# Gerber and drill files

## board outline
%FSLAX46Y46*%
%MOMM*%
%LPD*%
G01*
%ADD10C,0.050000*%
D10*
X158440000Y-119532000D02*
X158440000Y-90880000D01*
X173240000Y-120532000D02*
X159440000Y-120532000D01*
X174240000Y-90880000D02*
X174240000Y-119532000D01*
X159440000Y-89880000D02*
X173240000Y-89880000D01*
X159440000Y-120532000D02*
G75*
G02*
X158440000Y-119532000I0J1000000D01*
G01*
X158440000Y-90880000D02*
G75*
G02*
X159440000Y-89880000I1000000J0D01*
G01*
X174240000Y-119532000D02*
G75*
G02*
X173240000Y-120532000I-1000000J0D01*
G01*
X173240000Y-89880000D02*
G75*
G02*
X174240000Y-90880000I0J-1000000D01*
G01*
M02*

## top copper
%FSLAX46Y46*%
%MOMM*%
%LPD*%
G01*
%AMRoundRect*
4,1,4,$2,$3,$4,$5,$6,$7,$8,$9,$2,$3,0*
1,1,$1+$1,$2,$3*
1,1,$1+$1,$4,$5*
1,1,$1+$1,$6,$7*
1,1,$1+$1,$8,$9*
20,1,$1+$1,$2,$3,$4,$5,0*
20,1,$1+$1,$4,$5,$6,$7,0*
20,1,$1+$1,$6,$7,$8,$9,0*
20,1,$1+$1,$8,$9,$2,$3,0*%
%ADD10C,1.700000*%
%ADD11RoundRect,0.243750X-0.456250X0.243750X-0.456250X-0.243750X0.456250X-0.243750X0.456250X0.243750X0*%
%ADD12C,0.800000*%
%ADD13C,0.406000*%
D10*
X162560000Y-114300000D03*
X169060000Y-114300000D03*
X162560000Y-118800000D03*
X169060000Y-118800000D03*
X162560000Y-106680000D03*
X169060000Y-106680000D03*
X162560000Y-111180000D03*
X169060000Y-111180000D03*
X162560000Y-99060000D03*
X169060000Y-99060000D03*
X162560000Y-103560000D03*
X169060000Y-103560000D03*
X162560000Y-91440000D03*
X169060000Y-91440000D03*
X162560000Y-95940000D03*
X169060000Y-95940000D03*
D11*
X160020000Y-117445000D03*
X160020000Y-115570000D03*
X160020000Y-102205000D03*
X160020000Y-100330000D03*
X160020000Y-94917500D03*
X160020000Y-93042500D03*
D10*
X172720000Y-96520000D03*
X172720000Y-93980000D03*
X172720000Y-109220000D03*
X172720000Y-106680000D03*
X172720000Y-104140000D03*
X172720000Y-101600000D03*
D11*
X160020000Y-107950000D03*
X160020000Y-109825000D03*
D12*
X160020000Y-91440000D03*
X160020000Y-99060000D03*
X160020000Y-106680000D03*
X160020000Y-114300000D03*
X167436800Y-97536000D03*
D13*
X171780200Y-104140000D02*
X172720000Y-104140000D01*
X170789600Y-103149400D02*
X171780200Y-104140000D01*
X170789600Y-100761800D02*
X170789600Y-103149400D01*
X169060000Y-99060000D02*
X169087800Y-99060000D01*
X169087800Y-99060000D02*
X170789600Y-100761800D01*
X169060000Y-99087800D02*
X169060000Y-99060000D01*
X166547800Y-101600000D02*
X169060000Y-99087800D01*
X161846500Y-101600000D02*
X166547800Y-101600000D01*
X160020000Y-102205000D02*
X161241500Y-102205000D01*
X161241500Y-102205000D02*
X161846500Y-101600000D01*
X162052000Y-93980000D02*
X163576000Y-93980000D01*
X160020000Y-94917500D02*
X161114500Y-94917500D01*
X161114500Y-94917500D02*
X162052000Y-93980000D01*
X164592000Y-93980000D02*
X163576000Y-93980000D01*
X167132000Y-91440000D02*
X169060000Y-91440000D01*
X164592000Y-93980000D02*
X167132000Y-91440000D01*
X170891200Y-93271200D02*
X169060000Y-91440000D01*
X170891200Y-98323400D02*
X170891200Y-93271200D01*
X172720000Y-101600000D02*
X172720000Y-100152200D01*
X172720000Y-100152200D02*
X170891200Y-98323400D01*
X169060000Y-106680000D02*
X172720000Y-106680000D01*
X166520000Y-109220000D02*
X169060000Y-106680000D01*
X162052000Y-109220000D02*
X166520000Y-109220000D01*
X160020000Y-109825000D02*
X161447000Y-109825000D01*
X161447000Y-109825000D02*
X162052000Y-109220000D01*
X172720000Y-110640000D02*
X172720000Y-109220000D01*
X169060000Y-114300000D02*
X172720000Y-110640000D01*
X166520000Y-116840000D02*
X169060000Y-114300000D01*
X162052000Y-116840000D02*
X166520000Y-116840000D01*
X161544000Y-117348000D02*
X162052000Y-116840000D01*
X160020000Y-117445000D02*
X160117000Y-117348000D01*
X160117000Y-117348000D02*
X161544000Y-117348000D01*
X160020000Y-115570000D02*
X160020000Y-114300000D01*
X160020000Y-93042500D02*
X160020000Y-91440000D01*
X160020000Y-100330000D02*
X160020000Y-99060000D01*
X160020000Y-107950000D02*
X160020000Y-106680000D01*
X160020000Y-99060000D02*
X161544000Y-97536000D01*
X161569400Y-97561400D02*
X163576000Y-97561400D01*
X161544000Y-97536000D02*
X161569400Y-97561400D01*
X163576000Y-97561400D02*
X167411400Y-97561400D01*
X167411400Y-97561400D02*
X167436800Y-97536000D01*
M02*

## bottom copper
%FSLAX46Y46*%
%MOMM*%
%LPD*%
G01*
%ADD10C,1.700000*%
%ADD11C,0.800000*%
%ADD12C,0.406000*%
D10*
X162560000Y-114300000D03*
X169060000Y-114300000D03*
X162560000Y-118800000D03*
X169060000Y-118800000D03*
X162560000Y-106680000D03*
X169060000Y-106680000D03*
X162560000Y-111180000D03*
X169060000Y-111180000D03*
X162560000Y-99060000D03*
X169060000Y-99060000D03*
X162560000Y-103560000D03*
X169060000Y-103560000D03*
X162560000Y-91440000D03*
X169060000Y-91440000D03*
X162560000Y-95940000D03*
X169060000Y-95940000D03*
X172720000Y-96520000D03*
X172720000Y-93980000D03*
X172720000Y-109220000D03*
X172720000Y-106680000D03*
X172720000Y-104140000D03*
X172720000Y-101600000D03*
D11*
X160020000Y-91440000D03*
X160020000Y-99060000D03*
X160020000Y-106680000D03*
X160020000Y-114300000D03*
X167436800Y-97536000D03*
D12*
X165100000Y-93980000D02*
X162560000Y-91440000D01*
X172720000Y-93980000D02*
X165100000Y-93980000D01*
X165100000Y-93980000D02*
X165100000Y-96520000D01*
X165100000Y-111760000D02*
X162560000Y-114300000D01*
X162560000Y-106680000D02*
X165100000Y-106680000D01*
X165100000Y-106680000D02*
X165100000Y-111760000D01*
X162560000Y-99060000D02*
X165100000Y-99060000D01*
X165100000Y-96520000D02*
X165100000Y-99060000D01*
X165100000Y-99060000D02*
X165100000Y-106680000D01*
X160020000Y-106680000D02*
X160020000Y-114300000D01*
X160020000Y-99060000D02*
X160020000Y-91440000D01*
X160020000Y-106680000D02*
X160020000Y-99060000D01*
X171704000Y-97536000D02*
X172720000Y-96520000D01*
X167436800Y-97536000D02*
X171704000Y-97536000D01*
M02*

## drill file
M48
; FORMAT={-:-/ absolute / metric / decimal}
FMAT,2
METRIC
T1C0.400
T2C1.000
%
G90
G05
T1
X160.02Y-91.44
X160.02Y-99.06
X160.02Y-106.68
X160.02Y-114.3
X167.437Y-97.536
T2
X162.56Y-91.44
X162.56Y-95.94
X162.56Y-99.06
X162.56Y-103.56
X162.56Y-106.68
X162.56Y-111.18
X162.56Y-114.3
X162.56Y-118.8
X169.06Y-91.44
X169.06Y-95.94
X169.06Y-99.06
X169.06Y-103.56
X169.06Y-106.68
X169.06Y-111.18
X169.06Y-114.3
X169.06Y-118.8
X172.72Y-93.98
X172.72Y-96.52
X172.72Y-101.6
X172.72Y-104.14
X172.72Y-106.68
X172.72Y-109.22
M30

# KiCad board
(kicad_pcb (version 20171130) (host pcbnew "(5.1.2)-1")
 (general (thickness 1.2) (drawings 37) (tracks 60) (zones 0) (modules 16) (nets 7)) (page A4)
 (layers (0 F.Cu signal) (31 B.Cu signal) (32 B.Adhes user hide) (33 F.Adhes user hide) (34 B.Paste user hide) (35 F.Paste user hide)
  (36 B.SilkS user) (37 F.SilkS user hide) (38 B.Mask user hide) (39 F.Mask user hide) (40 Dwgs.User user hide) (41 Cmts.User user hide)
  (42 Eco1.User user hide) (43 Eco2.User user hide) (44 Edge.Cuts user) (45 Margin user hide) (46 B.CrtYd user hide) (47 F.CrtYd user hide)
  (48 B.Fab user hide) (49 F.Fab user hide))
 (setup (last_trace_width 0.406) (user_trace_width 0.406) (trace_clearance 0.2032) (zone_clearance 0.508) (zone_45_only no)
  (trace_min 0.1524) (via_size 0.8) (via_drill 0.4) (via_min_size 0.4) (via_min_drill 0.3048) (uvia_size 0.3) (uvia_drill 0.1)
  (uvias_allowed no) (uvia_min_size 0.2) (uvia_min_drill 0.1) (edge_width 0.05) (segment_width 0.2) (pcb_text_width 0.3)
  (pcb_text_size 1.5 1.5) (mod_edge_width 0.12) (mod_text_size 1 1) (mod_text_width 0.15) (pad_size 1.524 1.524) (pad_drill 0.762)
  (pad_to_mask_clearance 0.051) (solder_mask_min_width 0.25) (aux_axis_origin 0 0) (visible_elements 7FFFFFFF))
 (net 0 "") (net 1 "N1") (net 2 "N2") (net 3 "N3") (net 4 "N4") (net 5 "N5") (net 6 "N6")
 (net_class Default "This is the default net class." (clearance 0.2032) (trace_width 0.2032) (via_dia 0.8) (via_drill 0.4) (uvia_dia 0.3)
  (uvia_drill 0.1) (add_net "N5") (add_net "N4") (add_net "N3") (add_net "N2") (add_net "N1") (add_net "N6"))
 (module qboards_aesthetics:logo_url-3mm (layer B.Cu) (at 165.2778 94.742 270)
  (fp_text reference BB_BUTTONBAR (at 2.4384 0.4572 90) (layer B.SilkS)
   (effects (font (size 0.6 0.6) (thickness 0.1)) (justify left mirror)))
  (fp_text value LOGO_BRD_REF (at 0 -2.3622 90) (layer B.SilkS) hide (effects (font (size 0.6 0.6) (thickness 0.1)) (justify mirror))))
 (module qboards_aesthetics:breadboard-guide (layer F.Cu) (at 137.16 93.98)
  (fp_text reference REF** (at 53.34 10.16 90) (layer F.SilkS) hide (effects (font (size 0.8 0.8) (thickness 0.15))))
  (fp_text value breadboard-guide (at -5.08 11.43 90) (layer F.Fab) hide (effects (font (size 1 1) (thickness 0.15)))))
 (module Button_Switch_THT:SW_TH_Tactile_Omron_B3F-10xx (layer F.Cu) (at 162.56 114.3)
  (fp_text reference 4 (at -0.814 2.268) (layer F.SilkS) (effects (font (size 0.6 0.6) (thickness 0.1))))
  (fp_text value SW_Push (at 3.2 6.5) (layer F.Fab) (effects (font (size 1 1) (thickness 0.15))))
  (pad 1 thru_hole circle (at 0 0) (size 1.7 1.7) (drill 1) (layers *.Cu *.Mask) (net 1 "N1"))
  (pad 2 thru_hole circle (at 6.5 0) (size 1.7 1.7) (drill 1) (layers *.Cu *.Mask) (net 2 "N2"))
  (pad 3 thru_hole circle (at 0 4.5) (size 1.7 1.7) (drill 1) (layers *.Cu *.Mask))
  (pad 4 thru_hole circle (at 6.5 4.5) (size 1.7 1.7) (drill 1) (layers *.Cu *.Mask)))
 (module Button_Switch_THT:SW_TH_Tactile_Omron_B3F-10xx (layer F.Cu) (at 162.56 106.68)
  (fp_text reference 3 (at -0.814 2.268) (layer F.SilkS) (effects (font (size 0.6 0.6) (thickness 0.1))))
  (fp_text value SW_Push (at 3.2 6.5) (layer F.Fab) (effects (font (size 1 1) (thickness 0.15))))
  (pad 1 thru_hole circle (at 0 0) (size 1.7 1.7) (drill 1) (layers *.Cu *.Mask) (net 1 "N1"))
  (pad 2 thru_hole circle (at 6.5 0) (size 1.7 1.7) (drill 1) (layers *.Cu *.Mask) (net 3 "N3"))
  (pad 3 thru_hole circle (at 0 4.5) (size 1.7 1.7) (drill 1) (layers *.Cu *.Mask))
  (pad 4 thru_hole circle (at 6.5 4.5) (size 1.7 1.7) (drill 1) (layers *.Cu *.Mask)))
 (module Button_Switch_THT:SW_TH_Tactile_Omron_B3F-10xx (layer F.Cu) (at 162.56 99.06)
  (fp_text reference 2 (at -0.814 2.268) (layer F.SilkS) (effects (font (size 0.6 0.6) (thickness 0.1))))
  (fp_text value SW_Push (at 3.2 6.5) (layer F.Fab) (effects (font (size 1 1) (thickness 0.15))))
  (pad 1 thru_hole circle (at 0 0) (size 1.7 1.7) (drill 1) (layers *.Cu *.Mask) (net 1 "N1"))
  (pad 2 thru_hole circle (at 6.5 0) (size 1.7 1.7) (drill 1) (layers *.Cu *.Mask) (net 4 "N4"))
  (pad 3 thru_hole circle (at 0 4.5) (size 1.7 1.7) (drill 1) (layers *.Cu *.Mask))
  (pad 4 thru_hole circle (at 6.5 4.5) (size 1.7 1.7) (drill 1) (layers *.Cu *.Mask)))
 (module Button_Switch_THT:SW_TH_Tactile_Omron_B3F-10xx (layer F.Cu) (at 162.56 91.44)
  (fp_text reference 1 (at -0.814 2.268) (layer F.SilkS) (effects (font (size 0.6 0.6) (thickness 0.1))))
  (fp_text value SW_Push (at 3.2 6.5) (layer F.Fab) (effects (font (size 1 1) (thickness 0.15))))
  (pad 1 thru_hole circle (at 0 0) (size 1.7 1.7) (drill 1) (layers *.Cu *.Mask) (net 1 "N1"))
  (pad 2 thru_hole circle (at 6.5 0) (size 1.7 1.7) (drill 1) (layers *.Cu *.Mask) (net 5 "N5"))
  (pad 3 thru_hole circle (at 0 4.5) (size 1.7 1.7) (drill 1) (layers *.Cu *.Mask))
  (pad 4 thru_hole circle (at 6.5 4.5) (size 1.7 1.7) (drill 1) (layers *.Cu *.Mask)))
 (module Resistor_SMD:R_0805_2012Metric (layer F.Cu) (at 160.02 116.5075 270)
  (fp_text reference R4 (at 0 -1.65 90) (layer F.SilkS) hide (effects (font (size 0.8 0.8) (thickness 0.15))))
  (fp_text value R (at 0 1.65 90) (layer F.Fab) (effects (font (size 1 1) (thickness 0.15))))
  (pad 2 smd roundrect (at 0.9375 0 270) (size 0.975 1.4) (layers F.Cu F.Paste F.Mask) (roundrect_rratio 0.25) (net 2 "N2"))
  (pad 1 smd roundrect (at -0.9375 0 270) (size 0.975 1.4) (layers F.Cu F.Paste F.Mask) (roundrect_rratio 0.25) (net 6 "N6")))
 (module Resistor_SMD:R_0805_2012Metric (layer F.Cu) (at 160.02 101.2675 270)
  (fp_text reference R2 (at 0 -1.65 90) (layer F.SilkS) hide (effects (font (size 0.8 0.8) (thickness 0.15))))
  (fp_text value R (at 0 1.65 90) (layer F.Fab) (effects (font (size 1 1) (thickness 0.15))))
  (pad 2 smd roundrect (at 0.9375 0 270) (size 0.975 1.4) (layers F.Cu F.Paste F.Mask) (roundrect_rratio 0.25) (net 4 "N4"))
  (pad 1 smd roundrect (at -0.9375 0 270) (size 0.975 1.4) (layers F.Cu F.Paste F.Mask) (roundrect_rratio 0.25) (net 6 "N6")))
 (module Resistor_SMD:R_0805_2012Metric (layer F.Cu) (at 160.02 93.98 270)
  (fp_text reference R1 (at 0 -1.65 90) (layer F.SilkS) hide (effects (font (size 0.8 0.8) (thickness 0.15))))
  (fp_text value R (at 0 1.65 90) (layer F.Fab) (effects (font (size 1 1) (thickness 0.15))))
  (pad 2 smd roundrect (at 0.9375 0 270) (size 0.975 1.4) (layers F.Cu F.Paste F.Mask) (roundrect_rratio 0.25) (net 5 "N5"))
  (pad 1 smd roundrect (at -0.9375 0 270) (size 0.975 1.4) (layers F.Cu F.Paste F.Mask) (roundrect_rratio 0.25) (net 6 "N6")))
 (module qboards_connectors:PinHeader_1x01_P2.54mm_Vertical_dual (layer F.Cu) (at 172.72 96.52)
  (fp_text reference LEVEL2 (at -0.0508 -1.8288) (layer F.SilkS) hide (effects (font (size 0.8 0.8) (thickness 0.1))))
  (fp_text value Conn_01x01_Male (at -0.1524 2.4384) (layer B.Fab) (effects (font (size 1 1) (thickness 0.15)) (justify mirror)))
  (pad 1 thru_hole circle (at 0 0) (size 1.7 1.7) (drill 1) (layers *.Cu *.Mask) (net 6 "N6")))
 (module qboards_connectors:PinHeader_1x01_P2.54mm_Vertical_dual (layer F.Cu) (at 172.72 93.98)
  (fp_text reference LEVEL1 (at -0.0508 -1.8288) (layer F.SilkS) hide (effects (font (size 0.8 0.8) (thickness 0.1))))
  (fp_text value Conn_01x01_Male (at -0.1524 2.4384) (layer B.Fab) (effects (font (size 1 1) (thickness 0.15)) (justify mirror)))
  (pad 1 thru_hole circle (at 0 0) (size 1.7 1.7) (drill 1) (layers *.Cu *.Mask) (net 1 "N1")))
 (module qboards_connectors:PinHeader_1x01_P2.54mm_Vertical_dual (layer F.Cu) (at 172.72 109.22)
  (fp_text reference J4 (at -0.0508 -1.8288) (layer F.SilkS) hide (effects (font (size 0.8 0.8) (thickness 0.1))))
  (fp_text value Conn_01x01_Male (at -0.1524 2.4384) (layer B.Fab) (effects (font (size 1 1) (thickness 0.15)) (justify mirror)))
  (pad 1 thru_hole circle (at 0 0) (size 1.7 1.7) (drill 1) (layers *.Cu *.Mask) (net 2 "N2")))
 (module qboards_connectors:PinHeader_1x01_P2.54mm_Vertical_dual (layer F.Cu) (at 172.72 106.68)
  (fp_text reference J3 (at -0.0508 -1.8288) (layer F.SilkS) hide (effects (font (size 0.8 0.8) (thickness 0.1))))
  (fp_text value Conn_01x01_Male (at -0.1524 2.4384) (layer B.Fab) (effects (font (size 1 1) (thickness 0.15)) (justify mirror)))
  (pad 1 thru_hole circle (at 0 0) (size 1.7 1.7) (drill 1) (layers *.Cu *.Mask) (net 3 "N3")))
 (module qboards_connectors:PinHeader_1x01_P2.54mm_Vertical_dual (layer F.Cu) (at 172.72 104.14)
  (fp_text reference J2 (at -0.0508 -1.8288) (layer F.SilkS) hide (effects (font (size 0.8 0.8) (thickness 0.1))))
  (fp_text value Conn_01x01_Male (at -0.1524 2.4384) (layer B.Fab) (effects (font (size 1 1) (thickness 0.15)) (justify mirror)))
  (pad 1 thru_hole circle (at 0 0) (size 1.7 1.7) (drill 1) (layers *.Cu *.Mask) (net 4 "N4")))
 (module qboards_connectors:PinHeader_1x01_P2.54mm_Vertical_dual (layer F.Cu) (at 172.72 101.6)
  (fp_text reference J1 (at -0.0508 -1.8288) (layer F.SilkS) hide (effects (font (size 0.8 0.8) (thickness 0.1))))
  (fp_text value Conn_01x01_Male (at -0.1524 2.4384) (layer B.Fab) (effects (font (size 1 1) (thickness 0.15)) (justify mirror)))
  (pad 1 thru_hole circle (at 0 0) (size 1.7 1.7) (drill 1) (layers *.Cu *.Mask) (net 5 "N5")))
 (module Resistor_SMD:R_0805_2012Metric (layer F.Cu) (at 160.02 108.8875 270)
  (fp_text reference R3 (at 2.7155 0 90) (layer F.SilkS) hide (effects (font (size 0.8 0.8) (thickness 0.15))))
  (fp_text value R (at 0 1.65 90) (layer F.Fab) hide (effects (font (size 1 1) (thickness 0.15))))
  (pad 1 smd roundrect (at -0.9375 0 270) (size 0.975 1.4) (layers F.Cu F.Paste F.Mask) (roundrect_rratio 0.25) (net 6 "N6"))
  (pad 2 smd roundrect (at 0.9375 0 270) (size 0.975 1.4) (layers F.Cu F.Paste F.Mask) (roundrect_rratio 0.25) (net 3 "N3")))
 (gr_line (start 158.44 119.532) (end 158.44 90.88) (layer Edge.Cuts) (width 0.05))
 (gr_line (start 173.24 120.532) (end 159.44 120.532) (layer Edge.Cuts) (width 0.05))
 (gr_line (start 174.24 90.88) (end 174.24 119.532) (layer Edge.Cuts) (width 0.05))
 (gr_line (start 159.44 89.88) (end 173.24 89.88) (layer Edge.Cuts) (width 0.05))
 (gr_arc (start 159.44 119.532) (end 158.44 119.532) (angle -90) (layer Edge.Cuts) (width 0.05))
 (gr_arc (start 159.44 90.88) (end 159.44 89.88) (angle -90) (layer Edge.Cuts) (width 0.05))
 (gr_arc (start 173.24 119.532) (end 173.24 120.532) (angle -90) (layer Edge.Cuts) (width 0.05))
 (gr_arc (start 173.24 90.88) (end 174.24 90.88) (angle -90) (layer Edge.Cuts) (width 0.05))
 (segment (start 171.7802 104.14) (end 172.72 104.14) (width 0.406) (layer F.Cu) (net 4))
 (segment (start 170.7896 103.1494) (end 171.7802 104.14) (width 0.406) (layer F.Cu) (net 4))
 (segment (start 170.7896 100.7618) (end 170.7896 103.1494) (width 0.406) (layer F.Cu) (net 4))
 (segment (start 169.06 99.06) (end 169.0878 99.06) (width 0.406) (layer F.Cu) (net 4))
 (segment (start 169.0878 99.06) (end 170.7896 100.7618) (width 0.406) (layer F.Cu) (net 4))
 (segment (start 169.06 99.0878) (end 169.06 99.06) (width 0.406) (layer F.Cu) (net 4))
 (segment (start 166.5478 101.6) (end 169.06 99.0878) (width 0.406) (layer F.Cu) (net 4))
 (segment (start 161.8465 101.6) (end 166.5478 101.6) (width 0.406) (layer F.Cu) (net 4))
 (segment (start 160.02 102.205) (end 161.2415 102.205) (width 0.406) (layer F.Cu) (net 4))
 (segment (start 161.2415 102.205) (end 161.8465 101.6) (width 0.406) (layer F.Cu) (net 4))
 (segment (start 162.052 93.98) (end 163.576 93.98) (width 0.406) (layer F.Cu) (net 5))
 (segment (start 160.02 94.9175) (end 161.1145 94.9175) (width 0.406) (layer F.Cu) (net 5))
 (segment (start 161.1145 94.9175) (end 162.052 93.98) (width 0.406) (layer F.Cu) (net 5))
 (segment (start 164.592 93.98) (end 163.576 93.98) (width 0.406) (layer F.Cu) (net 5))
 (segment (start 167.132 91.44) (end 169.06 91.44) (width 0.406) (layer F.Cu) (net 5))
 (segment (start 164.592 93.98) (end 167.132 91.44) (width 0.406) (layer F.Cu) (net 5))
 (segment (start 170.8912 93.2712) (end 169.06 91.44) (width 0.406) (layer F.Cu) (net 5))
 (segment (start 170.8912 98.3234) (end 170.8912 93.2712) (width 0.406) (layer F.Cu) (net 5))
 (segment (start 172.72 101.6) (end 172.72 100.1522) (width 0.406) (layer F.Cu) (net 5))
 (segment (start 172.72 100.1522) (end 170.8912 98.3234) (width 0.406) (layer F.Cu) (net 5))
 (segment (start 169.06 106.68) (end 172.72 106.68) (width 0.406) (layer F.Cu) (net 3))
 (segment (start 166.52 109.22) (end 169.06 106.68) (width 0.406) (layer F.Cu) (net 3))
 (segment (start 162.052 109.22) (end 166.52 109.22) (width 0.406) (layer F.Cu) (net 3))
 (segment (start 160.02 109.825) (end 161.447 109.825) (width 0.406) (layer F.Cu) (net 3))
 (segment (start 161.447 109.825) (end 162.052 109.22) (width 0.406) (layer F.Cu) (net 3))
 (segment (start 172.72 110.64) (end 172.72 109.22) (width 0.406) (layer F.Cu) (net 2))
 (segment (start 169.06 114.3) (end 172.72 110.64) (width 0.406) (layer F.Cu) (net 2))
 (segment (start 166.52 116.84) (end 169.06 114.3) (width 0.406) (layer F.Cu) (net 2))
 (segment (start 162.052 116.84) (end 166.52 116.84) (width 0.406) (layer F.Cu) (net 2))
 (segment (start 161.544 117.348) (end 162.052 116.84) (width 0.406) (layer F.Cu) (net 2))
 (segment (start 160.02 117.445) (end 160.117 117.348) (width 0.406) (layer F.Cu) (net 2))
 (segment (start 160.117 117.348) (end 161.544 117.348) (width 0.406) (layer F.Cu) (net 2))
 (segment (start 165.1 93.98) (end 162.56 91.44) (width 0.406) (layer B.Cu) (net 1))
 (segment (start 172.72 93.98) (end 165.1 93.98) (width 0.406) (layer B.Cu) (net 1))
 (segment (start 165.1 93.98) (end 165.1 96.52) (width 0.406) (layer B.Cu) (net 1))
 (segment (start 165.1 111.76) (end 162.56 114.3) (width 0.406) (layer B.Cu) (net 1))
 (segment (start 162.56 106.68) (end 165.1 106.68) (width 0.406) (layer B.Cu) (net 1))
 (segment (start 165.1 106.68) (end 165.1 111.76) (width 0.406) (layer B.Cu) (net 1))
 (segment (start 162.56 99.06) (end 165.1 99.06) (width 0.406) (layer B.Cu) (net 1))
 (segment (start 165.1 96.52) (end 165.1 99.06) (width 0.406) (layer B.Cu) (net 1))
 (segment (start 165.1 99.06) (end 165.1 106.68) (width 0.406) (layer B.Cu) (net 1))
 (segment (start 160.02 115.57) (end 160.02 114.3) (width 0.406) (layer F.Cu) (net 6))
 (via (at 160.02 91.44) (size 0.8) (drill 0.4) (layers F.Cu B.Cu) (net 6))
 (segment (start 160.02 93.0425) (end 160.02 91.44) (width 0.406) (layer F.Cu) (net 6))
 (via (at 160.02 99.06) (size 0.8) (drill 0.4) (layers F.Cu B.Cu) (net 6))
 (segment (start 160.02 100.33) (end 160.02 99.06) (width 0.406) (layer F.Cu) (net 6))
 (via (at 160.02 106.68) (size 0.8) (drill 0.4) (layers F.Cu B.Cu) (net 6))
 (segment (start 160.02 107.95) (end 160.02 106.68) (width 0.406) (layer F.Cu) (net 6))
 (segment (start 160.02 106.68) (end 160.02 114.3) (width 0.406) (layer B.Cu) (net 6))
 (via (at 160.02 114.3) (size 0.8) (drill 0.4) (layers F.Cu B.Cu) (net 6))
 (segment (start 160.02 99.06) (end 160.02 91.44) (width 0.406) (layer B.Cu) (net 6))
 (segment (start 160.02 106.68) (end 160.02 99.06) (width 0.406) (layer B.Cu) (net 6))
 (segment (start 160.02 99.06) (end 161.544 97.536) (width 0.406) (layer F.Cu) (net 6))
 (segment (start 161.5694 97.5614) (end 163.576 97.5614) (width 0.406) (layer F.Cu) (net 6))
 (segment (start 161.544 97.536) (end 161.5694 97.5614) (width 0.406) (layer F.Cu) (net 6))
 (via (at 167.4368 97.536) (size 0.8) (drill 0.4) (layers F.Cu B.Cu) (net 6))
 (segment (start 163.576 97.5614) (end 167.4114 97.5614) (width 0.406) (layer F.Cu) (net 6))
 (segment (start 167.4114 97.5614) (end 167.4368 97.536) (width 0.406) (layer F.Cu) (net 6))
 (segment (start 171.704 97.536) (end 172.72 96.52) (width 0.406) (layer B.Cu) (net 6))
 (segment (start 167.4368 97.536) (end 171.704 97.536) (width 0.406) (layer B.Cu) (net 6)))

